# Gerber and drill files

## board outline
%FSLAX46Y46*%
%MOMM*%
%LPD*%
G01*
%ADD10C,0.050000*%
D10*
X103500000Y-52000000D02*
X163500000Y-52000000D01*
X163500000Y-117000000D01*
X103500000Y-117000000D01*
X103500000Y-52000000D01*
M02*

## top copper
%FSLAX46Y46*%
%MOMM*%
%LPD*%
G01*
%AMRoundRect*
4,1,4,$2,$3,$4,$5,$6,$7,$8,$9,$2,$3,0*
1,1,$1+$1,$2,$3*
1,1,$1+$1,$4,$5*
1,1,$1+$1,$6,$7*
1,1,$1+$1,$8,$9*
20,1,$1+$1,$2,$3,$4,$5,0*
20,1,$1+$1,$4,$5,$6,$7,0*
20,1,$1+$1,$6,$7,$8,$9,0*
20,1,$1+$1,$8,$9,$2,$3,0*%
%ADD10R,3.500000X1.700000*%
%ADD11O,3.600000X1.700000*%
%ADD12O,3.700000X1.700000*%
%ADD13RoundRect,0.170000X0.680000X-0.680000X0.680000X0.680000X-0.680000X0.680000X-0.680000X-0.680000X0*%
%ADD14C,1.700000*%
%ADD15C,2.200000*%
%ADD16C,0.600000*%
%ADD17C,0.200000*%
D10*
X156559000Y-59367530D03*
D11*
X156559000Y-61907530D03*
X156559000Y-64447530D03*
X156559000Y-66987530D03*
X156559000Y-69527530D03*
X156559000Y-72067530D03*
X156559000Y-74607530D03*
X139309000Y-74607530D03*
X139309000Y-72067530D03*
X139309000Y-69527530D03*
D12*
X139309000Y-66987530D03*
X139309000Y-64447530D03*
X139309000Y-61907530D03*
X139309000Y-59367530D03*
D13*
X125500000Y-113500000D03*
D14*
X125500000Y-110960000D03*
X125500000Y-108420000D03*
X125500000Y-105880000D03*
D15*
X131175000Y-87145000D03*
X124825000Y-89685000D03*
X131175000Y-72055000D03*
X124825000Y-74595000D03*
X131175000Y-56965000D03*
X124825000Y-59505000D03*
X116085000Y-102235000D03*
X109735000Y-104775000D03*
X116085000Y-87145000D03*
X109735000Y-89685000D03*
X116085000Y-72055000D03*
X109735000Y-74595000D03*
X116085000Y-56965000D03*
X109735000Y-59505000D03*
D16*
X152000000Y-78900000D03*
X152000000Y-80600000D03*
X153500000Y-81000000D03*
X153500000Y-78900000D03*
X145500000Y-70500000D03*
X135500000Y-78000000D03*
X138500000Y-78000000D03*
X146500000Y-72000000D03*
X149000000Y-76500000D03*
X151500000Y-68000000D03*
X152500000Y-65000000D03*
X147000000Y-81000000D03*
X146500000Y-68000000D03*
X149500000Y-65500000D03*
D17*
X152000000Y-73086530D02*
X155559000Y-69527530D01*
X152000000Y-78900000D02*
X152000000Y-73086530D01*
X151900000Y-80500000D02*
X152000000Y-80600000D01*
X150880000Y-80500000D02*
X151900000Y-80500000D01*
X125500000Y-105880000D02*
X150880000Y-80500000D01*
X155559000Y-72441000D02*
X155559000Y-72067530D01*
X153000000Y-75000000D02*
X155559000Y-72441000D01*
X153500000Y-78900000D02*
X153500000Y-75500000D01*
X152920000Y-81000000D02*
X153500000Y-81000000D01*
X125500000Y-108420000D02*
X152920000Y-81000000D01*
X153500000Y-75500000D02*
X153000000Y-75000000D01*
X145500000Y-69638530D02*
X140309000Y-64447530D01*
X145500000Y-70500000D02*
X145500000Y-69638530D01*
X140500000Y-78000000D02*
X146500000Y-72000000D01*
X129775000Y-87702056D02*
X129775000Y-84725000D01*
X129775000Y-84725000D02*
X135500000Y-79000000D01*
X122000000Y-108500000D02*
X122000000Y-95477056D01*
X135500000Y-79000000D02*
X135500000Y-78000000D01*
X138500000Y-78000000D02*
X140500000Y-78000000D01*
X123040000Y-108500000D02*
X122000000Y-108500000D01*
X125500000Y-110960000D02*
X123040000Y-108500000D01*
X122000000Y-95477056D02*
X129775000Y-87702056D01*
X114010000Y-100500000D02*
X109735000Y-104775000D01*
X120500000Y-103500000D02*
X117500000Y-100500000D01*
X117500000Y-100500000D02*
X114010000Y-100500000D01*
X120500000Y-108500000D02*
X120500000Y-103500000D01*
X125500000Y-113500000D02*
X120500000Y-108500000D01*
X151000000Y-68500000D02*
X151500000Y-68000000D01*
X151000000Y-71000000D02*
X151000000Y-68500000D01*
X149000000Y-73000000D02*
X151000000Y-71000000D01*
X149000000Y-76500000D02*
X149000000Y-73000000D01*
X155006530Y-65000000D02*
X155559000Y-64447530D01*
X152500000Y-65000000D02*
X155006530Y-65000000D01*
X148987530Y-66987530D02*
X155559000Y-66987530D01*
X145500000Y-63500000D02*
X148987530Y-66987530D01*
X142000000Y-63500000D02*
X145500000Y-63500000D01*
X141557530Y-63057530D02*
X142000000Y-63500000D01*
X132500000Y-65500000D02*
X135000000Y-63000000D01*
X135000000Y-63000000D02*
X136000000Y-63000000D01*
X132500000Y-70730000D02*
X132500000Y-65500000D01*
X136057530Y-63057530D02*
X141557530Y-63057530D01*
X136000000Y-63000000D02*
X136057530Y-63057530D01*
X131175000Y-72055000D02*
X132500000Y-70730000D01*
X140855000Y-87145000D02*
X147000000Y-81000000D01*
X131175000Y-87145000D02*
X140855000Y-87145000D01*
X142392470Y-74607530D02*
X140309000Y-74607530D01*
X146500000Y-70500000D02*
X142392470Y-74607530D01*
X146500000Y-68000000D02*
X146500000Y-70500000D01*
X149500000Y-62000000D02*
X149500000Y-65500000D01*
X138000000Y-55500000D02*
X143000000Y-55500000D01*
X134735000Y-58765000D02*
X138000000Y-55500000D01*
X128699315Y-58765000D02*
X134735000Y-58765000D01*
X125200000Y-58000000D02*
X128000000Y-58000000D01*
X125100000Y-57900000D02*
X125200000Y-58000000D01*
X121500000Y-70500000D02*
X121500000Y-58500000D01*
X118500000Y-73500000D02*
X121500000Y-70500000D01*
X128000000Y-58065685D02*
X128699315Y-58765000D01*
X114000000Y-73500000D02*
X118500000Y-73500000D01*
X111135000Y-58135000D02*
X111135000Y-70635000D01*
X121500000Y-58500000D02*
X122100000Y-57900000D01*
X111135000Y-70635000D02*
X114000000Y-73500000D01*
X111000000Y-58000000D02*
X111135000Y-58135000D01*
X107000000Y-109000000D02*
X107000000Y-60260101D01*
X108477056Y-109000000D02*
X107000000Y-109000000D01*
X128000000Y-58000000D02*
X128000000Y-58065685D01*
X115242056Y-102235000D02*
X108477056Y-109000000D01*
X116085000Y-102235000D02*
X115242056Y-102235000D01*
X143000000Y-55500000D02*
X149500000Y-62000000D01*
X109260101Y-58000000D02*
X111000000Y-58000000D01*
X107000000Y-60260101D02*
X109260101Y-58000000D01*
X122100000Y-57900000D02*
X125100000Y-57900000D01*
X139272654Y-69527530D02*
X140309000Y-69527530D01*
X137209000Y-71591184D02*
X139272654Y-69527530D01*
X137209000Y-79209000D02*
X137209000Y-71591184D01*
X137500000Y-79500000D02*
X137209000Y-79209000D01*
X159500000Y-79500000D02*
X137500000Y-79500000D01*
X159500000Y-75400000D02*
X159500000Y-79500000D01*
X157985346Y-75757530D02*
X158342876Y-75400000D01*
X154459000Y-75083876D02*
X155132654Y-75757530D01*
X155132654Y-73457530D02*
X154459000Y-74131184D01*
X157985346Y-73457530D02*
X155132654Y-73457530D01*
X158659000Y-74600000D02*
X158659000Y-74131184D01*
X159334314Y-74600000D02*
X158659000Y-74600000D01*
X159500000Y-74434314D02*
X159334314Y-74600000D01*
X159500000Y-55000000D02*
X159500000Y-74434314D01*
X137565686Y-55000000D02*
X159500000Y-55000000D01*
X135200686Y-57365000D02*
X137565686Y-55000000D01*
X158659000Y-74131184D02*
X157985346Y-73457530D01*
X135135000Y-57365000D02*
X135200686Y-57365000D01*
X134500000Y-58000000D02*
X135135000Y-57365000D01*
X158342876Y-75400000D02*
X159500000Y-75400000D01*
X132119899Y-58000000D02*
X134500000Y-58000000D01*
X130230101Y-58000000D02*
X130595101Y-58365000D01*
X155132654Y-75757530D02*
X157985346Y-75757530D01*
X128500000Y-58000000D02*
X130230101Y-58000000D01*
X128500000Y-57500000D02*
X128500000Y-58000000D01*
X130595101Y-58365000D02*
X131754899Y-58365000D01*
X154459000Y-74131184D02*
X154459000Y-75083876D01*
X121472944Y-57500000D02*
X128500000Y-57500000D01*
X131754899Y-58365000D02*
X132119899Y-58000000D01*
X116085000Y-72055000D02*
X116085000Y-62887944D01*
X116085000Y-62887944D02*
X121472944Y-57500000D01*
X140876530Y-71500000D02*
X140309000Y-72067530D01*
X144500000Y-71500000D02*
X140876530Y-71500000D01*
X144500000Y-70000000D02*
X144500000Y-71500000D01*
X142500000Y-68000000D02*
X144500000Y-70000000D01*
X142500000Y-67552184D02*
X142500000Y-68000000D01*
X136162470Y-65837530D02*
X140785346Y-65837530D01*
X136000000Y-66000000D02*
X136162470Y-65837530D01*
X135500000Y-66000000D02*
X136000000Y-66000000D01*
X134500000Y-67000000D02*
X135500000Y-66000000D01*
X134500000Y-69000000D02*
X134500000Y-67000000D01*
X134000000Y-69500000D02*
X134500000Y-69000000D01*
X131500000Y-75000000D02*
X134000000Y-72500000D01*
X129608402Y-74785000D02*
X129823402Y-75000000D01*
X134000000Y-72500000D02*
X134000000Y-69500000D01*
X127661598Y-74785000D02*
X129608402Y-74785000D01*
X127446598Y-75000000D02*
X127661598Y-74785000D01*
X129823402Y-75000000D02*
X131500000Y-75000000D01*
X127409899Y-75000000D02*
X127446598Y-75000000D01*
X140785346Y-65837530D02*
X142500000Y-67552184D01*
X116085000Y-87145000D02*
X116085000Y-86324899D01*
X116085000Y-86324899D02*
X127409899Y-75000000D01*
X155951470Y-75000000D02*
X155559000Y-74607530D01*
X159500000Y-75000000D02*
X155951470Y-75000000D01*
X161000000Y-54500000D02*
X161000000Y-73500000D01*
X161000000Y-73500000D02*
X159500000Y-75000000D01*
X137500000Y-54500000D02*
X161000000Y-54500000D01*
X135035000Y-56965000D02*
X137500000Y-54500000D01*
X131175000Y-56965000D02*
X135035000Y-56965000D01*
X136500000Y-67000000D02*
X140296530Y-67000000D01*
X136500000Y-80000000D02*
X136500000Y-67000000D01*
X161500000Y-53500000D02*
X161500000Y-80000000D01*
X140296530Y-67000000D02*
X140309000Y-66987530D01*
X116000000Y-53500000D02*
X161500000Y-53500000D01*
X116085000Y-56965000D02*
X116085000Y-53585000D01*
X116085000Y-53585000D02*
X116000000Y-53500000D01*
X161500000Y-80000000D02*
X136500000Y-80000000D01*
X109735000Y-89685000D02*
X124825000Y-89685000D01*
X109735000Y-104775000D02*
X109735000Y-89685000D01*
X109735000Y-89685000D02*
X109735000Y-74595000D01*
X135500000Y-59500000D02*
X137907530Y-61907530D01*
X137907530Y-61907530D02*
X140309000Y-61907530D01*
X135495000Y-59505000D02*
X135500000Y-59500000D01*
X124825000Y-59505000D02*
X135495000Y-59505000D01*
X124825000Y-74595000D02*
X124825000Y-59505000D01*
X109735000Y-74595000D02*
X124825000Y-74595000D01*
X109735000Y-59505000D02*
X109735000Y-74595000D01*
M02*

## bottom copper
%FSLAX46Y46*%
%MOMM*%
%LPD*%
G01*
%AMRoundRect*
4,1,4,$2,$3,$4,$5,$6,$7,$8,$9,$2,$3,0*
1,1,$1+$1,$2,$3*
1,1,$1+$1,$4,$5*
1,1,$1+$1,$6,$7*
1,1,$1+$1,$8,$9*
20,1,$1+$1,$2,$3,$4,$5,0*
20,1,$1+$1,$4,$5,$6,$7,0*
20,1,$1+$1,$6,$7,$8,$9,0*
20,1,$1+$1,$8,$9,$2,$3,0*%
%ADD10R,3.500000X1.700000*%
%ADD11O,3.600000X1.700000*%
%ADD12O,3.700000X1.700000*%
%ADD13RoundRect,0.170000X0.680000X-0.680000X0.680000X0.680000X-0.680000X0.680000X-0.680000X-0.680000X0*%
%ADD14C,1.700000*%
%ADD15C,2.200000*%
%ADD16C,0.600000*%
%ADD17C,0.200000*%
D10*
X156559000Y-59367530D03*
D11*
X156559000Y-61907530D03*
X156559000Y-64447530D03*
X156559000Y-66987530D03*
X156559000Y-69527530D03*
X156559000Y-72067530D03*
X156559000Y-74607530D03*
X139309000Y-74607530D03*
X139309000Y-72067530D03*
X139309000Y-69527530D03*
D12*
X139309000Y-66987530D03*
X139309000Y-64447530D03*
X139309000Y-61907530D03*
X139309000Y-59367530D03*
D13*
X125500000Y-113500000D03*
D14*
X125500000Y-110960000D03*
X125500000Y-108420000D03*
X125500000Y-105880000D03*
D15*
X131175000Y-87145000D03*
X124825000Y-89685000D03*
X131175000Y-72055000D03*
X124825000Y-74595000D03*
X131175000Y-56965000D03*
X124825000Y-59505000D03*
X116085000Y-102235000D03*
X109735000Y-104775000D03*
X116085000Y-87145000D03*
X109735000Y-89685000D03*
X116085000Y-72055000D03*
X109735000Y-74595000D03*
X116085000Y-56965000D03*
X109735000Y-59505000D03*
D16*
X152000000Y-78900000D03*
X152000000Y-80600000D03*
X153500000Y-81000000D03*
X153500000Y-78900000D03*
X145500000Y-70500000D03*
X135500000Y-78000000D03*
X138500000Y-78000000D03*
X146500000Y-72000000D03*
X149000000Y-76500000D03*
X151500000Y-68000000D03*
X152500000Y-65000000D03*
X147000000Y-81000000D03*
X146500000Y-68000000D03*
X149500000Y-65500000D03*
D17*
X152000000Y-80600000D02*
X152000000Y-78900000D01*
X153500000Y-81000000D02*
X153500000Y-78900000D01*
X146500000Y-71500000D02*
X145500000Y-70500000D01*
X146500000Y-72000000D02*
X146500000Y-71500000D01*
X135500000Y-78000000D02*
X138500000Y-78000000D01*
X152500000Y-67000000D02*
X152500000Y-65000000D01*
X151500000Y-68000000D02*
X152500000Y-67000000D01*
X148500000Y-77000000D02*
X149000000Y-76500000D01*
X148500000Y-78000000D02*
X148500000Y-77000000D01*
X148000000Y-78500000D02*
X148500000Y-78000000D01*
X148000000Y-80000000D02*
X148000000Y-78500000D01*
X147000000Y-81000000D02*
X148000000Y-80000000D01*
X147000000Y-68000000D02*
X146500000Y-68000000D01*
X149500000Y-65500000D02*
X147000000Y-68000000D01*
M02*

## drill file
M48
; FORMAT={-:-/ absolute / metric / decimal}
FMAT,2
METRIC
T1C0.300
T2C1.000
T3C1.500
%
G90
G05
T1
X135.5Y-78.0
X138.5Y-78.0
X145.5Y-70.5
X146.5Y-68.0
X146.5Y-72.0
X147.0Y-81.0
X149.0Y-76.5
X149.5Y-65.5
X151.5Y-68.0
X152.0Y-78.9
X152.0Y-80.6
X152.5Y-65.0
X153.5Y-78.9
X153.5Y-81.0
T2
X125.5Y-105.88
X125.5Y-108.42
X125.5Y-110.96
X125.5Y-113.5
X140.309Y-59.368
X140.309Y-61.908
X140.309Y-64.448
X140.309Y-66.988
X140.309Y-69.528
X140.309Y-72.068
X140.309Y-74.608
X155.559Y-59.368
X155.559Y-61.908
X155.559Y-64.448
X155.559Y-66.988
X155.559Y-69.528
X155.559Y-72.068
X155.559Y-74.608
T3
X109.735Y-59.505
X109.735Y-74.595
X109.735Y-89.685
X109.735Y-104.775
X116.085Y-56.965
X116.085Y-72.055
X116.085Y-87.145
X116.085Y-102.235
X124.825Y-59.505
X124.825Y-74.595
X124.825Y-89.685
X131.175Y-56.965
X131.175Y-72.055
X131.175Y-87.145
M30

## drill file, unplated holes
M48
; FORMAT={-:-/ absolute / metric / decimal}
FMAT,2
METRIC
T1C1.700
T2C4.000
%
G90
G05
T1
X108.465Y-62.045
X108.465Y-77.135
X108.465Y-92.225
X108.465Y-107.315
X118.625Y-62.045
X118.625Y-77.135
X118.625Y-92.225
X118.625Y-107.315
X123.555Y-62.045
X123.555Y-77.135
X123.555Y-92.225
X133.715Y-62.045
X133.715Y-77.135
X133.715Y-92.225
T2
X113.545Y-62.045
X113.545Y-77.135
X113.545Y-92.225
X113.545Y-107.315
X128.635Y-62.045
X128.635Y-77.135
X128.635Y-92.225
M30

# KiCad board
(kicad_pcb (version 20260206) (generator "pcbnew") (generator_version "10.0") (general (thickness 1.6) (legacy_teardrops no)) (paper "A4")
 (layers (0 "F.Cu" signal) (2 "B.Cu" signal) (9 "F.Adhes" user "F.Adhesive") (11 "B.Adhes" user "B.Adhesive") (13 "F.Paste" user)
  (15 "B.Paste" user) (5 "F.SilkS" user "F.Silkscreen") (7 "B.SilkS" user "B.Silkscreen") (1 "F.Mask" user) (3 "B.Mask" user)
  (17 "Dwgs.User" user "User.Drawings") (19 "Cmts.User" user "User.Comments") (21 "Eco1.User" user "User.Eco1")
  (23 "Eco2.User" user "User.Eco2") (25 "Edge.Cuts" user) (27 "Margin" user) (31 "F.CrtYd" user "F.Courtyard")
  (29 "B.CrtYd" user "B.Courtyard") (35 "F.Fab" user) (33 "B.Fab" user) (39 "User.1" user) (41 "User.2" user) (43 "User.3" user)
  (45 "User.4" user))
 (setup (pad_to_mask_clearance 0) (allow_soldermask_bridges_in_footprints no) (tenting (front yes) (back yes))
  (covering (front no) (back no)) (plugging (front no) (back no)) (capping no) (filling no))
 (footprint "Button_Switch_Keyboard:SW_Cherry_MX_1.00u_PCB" (layer "F.Cu") (at 131.175 56.965)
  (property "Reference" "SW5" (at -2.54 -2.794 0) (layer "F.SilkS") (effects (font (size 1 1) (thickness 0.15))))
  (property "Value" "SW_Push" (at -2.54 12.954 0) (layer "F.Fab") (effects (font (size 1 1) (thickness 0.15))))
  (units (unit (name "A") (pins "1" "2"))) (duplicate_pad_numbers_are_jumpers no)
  (pad "" np_thru_hole circle (at -7.62 5.08) (size 1.7 1.7) (drill 1.7) (layers "*.Cu" "*.Mask"))
  (pad "" np_thru_hole circle (at -2.54 5.08) (size 4 4) (drill 4) (layers "*.Cu" "*.Mask"))
  (pad "" np_thru_hole circle (at 2.54 5.08) (size 1.7 1.7) (drill 1.7) (layers "*.Cu" "*.Mask"))
  (pad "1" thru_hole circle (at 0 0) (size 2.2 2.2) (drill 1.5) (layers "*.Cu" "*.Mask") (remove_unused_layers no)
   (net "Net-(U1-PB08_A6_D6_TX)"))
  (pad "2" thru_hole circle (at -6.35 2.54) (size 2.2 2.2) (drill 1.5) (layers "*.Cu" "*.Mask") (remove_unused_layers no) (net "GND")))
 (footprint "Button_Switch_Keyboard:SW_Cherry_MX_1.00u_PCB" (layer "F.Cu") (at 116.085 72.055)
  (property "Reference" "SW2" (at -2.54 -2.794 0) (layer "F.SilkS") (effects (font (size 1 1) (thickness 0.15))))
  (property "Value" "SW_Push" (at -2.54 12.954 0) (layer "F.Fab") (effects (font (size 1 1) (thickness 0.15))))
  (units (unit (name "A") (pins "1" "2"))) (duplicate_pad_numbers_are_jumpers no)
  (pad "" np_thru_hole circle (at -7.62 5.08) (size 1.7 1.7) (drill 1.7) (layers "*.Cu" "*.Mask"))
  (pad "" np_thru_hole circle (at -2.54 5.08) (size 4 4) (drill 4) (layers "*.Cu" "*.Mask"))
  (pad "" np_thru_hole circle (at 2.54 5.08) (size 1.7 1.7) (drill 1.7) (layers "*.Cu" "*.Mask"))
  (pad "1" thru_hole circle (at 0 0) (size 2.2 2.2) (drill 1.5) (layers "*.Cu" "*.Mask") (remove_unused_layers no)
   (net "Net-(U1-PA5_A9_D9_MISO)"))
  (pad "2" thru_hole circle (at -6.35 2.54) (size 2.2 2.2) (drill 1.5) (layers "*.Cu" "*.Mask") (remove_unused_layers no) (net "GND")))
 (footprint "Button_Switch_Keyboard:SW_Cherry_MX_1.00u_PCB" (layer "F.Cu") (at 116.085 56.965)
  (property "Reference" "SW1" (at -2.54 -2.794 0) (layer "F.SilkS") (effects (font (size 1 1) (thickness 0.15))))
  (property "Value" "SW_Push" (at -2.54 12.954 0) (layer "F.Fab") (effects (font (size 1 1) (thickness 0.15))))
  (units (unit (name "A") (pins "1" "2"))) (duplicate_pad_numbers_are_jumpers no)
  (pad "" np_thru_hole circle (at -7.62 5.08) (size 1.7 1.7) (drill 1.7) (layers "*.Cu" "*.Mask"))
  (pad "" np_thru_hole circle (at -2.54 5.08) (size 4 4) (drill 4) (layers "*.Cu" "*.Mask"))
  (pad "" np_thru_hole circle (at 2.54 5.08) (size 1.7 1.7) (drill 1.7) (layers "*.Cu" "*.Mask"))
  (pad "1" thru_hole circle (at 0 0) (size 2.2 2.2) (drill 1.5) (layers "*.Cu" "*.Mask") (remove_unused_layers no)
   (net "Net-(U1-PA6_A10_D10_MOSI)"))
  (pad "2" thru_hole circle (at -6.35 2.54) (size 2.2 2.2) (drill 1.5) (layers "*.Cu" "*.Mask") (remove_unused_layers no) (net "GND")))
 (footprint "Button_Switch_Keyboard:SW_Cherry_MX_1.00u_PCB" (layer "F.Cu") (at 131.175 87.145)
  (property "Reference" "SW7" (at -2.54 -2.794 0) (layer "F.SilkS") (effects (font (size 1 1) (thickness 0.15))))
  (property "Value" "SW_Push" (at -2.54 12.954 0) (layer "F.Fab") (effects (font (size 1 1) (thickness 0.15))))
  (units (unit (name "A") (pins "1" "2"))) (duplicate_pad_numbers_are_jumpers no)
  (pad "" np_thru_hole circle (at -7.62 5.08) (size 1.7 1.7) (drill 1.7) (layers "*.Cu" "*.Mask"))
  (pad "" np_thru_hole circle (at -2.54 5.08) (size 4 4) (drill 4) (layers "*.Cu" "*.Mask"))
  (pad "" np_thru_hole circle (at 2.54 5.08) (size 1.7 1.7) (drill 1.7) (layers "*.Cu" "*.Mask"))
  (pad "1" thru_hole circle (at 0 0) (size 2.2 2.2) (drill 1.5) (layers "*.Cu" "*.Mask") (remove_unused_layers no)
   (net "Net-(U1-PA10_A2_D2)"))
  (pad "2" thru_hole circle (at -6.35 2.54) (size 2.2 2.2) (drill 1.5) (layers "*.Cu" "*.Mask") (remove_unused_layers no) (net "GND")))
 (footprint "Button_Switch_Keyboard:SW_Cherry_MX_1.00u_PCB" (layer "F.Cu") (at 116.085 102.235)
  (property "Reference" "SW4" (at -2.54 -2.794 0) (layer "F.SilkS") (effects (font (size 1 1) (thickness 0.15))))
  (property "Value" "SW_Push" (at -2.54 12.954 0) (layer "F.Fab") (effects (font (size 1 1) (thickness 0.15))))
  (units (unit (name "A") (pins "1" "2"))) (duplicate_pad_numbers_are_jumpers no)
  (pad "" np_thru_hole circle (at -7.62 5.08) (size 1.7 1.7) (drill 1.7) (layers "*.Cu" "*.Mask"))
  (pad "" np_thru_hole circle (at -2.54 5.08) (size 4 4) (drill 4) (layers "*.Cu" "*.Mask"))
  (pad "" np_thru_hole circle (at 2.54 5.08) (size 1.7 1.7) (drill 1.7) (layers "*.Cu" "*.Mask"))
  (pad "1" thru_hole circle (at 0 0) (size 2.2 2.2) (drill 1.5) (layers "*.Cu" "*.Mask") (remove_unused_layers no)
   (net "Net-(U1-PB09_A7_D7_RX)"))
  (pad "2" thru_hole circle (at -6.35 2.54) (size 2.2 2.2) (drill 1.5) (layers "*.Cu" "*.Mask") (remove_unused_layers no) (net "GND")))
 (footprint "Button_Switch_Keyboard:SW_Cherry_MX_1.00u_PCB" (layer "F.Cu") (at 131.175 72.055)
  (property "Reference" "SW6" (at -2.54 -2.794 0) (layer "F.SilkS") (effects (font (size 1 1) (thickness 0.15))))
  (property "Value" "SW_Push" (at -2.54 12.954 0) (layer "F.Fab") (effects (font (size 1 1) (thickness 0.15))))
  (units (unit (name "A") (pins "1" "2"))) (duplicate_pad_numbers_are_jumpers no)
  (pad "" np_thru_hole circle (at -7.62 5.08) (size 1.7 1.7) (drill 1.7) (layers "*.Cu" "*.Mask"))
  (pad "" np_thru_hole circle (at -2.54 5.08) (size 4 4) (drill 4) (layers "*.Cu" "*.Mask"))
  (pad "" np_thru_hole circle (at 2.54 5.08) (size 1.7 1.7) (drill 1.7) (layers "*.Cu" "*.Mask"))
  (pad "1" thru_hole circle (at 0 0) (size 2.2 2.2) (drill 1.5) (layers "*.Cu" "*.Mask") (remove_unused_layers no)
   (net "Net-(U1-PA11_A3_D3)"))
  (pad "2" thru_hole circle (at -6.35 2.54) (size 2.2 2.2) (drill 1.5) (layers "*.Cu" "*.Mask") (remove_unused_layers no) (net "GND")))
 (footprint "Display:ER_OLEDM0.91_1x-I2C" (layer "F.Cu") (at 125.5 113.5 90)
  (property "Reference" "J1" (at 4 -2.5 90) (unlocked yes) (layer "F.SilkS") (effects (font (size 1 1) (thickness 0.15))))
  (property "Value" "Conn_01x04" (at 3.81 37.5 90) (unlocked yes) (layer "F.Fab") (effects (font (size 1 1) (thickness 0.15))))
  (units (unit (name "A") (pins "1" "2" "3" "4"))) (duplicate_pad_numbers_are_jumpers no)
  (pad "1" thru_hole roundrect (at 0 0 90) (size 1.7 1.7) (drill 1) (layers "*.Cu" "*.Mask") (remove_unused_layers no)
   (roundrect_rratio 0.1) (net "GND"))
  (pad "2" thru_hole circle (at 2.54 0 90) (size 1.7 1.7) (drill 1) (layers "*.Cu" "*.Mask") (remove_unused_layers no)
   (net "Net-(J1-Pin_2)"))
  (pad "3" thru_hole circle (at 5.08 0 90) (size 1.7 1.7) (drill 1) (layers "*.Cu" "*.Mask") (remove_unused_layers no)
   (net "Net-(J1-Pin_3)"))
  (pad "4" thru_hole circle (at 7.62 0 90) (size 1.7 1.7) (drill 1) (layers "*.Cu" "*.Mask") (remove_unused_layers no)
   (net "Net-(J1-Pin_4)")))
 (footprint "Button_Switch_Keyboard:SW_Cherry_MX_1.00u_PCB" (layer "F.Cu") (at 116.085 87.145)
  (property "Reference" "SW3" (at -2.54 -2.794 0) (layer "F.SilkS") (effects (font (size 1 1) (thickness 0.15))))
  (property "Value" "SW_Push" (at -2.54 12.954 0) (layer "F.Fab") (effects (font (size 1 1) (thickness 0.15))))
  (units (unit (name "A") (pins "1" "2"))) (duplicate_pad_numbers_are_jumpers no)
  (pad "" np_thru_hole circle (at -7.62 5.08) (size 1.7 1.7) (drill 1.7) (layers "*.Cu" "*.Mask"))
  (pad "" np_thru_hole circle (at -2.54 5.08) (size 4 4) (drill 4) (layers "*.Cu" "*.Mask"))
  (pad "" np_thru_hole circle (at 2.54 5.08) (size 1.7 1.7) (drill 1.7) (layers "*.Cu" "*.Mask"))
  (pad "1" thru_hole circle (at 0 0) (size 2.2 2.2) (drill 1.5) (layers "*.Cu" "*.Mask") (remove_unused_layers no)
   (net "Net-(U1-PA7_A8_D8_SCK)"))
  (pad "2" thru_hole circle (at -6.35 2.54) (size 2.2 2.2) (drill 1.5) (layers "*.Cu" "*.Mask") (remove_unused_layers no) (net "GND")))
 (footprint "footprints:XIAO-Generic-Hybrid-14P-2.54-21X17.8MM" (layer "B.Cu") (at 147.934 66.98753 180)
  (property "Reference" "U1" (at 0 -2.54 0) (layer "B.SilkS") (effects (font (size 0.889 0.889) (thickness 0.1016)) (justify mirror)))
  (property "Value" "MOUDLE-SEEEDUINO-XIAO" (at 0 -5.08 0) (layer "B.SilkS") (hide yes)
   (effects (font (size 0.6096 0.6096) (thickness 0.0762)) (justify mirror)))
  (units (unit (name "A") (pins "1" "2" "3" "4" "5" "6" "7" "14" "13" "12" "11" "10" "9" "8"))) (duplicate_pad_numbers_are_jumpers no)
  (pad "1" thru_hole rect (at -7.625 7.62 180) (size 3.5 1.7) (drill 1 (offset -1 0)) (layers "*.Cu" "*.Mask") (remove_unused_layers no)
   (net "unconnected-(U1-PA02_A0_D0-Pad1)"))
  (pad "2" thru_hole oval (at -7.625 5.08 180) (size 3.6 1.7) (drill 1 (offset -1 0)) (layers "*.Cu" "*.Mask") (remove_unused_layers no)
   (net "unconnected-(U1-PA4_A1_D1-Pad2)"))
  (pad "3" thru_hole oval (at -7.625 2.54 180) (size 3.6 1.7) (drill 1 (offset -1 0)) (layers "*.Cu" "*.Mask") (remove_unused_layers no)
   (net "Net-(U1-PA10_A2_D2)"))
  (pad "4" thru_hole oval (at -7.625 0 180) (size 3.6 1.7) (drill 1 (offset -1 0)) (layers "*.Cu" "*.Mask") (remove_unused_layers no)
   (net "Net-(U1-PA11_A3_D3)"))
  (pad "5" thru_hole oval (at -7.625 -2.54 180) (size 3.6 1.7) (drill 1 (offset -1 0)) (layers "*.Cu" "*.Mask") (remove_unused_layers no)
   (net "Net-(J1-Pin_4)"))
  (pad "6" thru_hole oval (at -7.625 -5.08) (size 3.6 1.7) (drill 1 (offset 1 0)) (layers "*.Cu" "*.Mask") (remove_unused_layers no)
   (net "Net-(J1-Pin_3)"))
  (pad "7" thru_hole oval (at -7.625 -7.62 180) (size 3.6 1.7) (drill 1 (offset -1 0)) (layers "*.Cu" "*.Mask") (remove_unused_layers no)
   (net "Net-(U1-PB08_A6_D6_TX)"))
  (pad "8" thru_hole oval (at 7.625 -7.62 180) (size 3.6 1.7) (drill 1 (offset 1 0)) (layers "*.Cu" "*.Mask") (remove_unused_layers no)
   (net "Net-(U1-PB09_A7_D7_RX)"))
  (pad "9" thru_hole oval (at 7.625 -5.08 180) (size 3.6 1.7) (drill 1 (offset 1 0)) (layers "*.Cu" "*.Mask") (remove_unused_layers no)
   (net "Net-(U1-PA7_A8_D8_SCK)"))
  (pad "10" thru_hole oval (at 7.625 -2.54 180) (size 3.6 1.7) (drill 1 (offset 1 0)) (layers "*.Cu" "*.Mask") (remove_unused_layers no)
   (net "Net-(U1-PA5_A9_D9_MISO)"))
  (pad "11" thru_hole oval (at 7.625 0 180) (size 3.7 1.7) (drill 1 (offset 1 0)) (layers "*.Cu" "*.Mask") (remove_unused_layers no)
   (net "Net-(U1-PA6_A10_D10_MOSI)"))
  (pad "12" thru_hole oval (at 7.625 2.54 180) (size 3.7 1.7) (drill 1 (offset 1 0)) (layers "*.Cu" "*.Mask") (remove_unused_layers no)
   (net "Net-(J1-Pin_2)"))
  (pad "13" thru_hole oval (at 7.625 5.08 180) (size 3.7 1.7) (drill 1 (offset 1 0)) (layers "*.Cu" "*.Mask") (remove_unused_layers no)
   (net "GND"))
  (pad "14" thru_hole oval (at 7.625 7.62 180) (size 3.7 1.7) (drill 1 (offset 1 0)) (layers "*.Cu" "*.Mask") (remove_unused_layers no)
   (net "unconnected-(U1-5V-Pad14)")))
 (gr_rect (start 103.5 52) (end 163.5 117) (stroke (width 0.05) (type default)) (fill no) (layer "Edge.Cuts"))
 (segment (start 114.01 100.5) (end 109.735 104.775) (width 0.2) (layer "F.Cu") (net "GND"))
 (segment (start 109.735 89.685) (end 124.825 89.685) (width 0.2) (layer "F.Cu") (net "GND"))
 (segment (start 135.495 59.505) (end 135.5 59.5) (width 0.2) (layer "F.Cu") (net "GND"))
 (segment (start 125.5 113.5) (end 120.5 108.5) (width 0.2) (layer "F.Cu") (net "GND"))
 (segment (start 124.825 59.505) (end 135.495 59.505) (width 0.2) (layer "F.Cu") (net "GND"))
 (segment (start 117.5 100.5) (end 114.01 100.5) (width 0.2) (layer "F.Cu") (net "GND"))
 (segment (start 120.5 108.5) (end 120.5 103.5) (width 0.2) (layer "F.Cu") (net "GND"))
 (segment (start 109.735 59.505) (end 109.735 74.595) (width 0.2) (layer "F.Cu") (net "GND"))
 (segment (start 135.5 59.5) (end 137.90753 61.90753) (width 0.2) (layer "F.Cu") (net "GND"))
 (segment (start 137.90753 61.90753) (end 140.309 61.90753) (width 0.2) (layer "F.Cu") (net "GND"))
 (segment (start 109.735 74.595) (end 124.825 74.595) (width 0.2) (layer "F.Cu") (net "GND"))
 (segment (start 109.735 104.775) (end 109.735 89.685) (width 0.2) (layer "F.Cu") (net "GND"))
 (segment (start 109.735 89.685) (end 109.735 74.595) (width 0.2) (layer "F.Cu") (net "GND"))
 (segment (start 120.5 103.5) (end 117.5 100.5) (width 0.2) (layer "F.Cu") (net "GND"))
 (segment (start 124.825 74.595) (end 124.825 59.505) (width 0.2) (layer "F.Cu") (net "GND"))
 (segment (start 161.5 53.5) (end 161.5 80) (width 0.2) (layer "F.Cu") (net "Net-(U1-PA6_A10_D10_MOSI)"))
 (segment (start 136.5 80) (end 136.5 67) (width 0.2) (layer "F.Cu") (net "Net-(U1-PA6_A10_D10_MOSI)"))
 (segment (start 140.29653 67) (end 140.309 66.98753) (width 0.2) (layer "F.Cu") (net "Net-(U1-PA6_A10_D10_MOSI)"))
 (segment (start 116.085 53.585) (end 116 53.5) (width 0.2) (layer "F.Cu") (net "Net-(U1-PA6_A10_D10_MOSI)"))
 (segment (start 136.5 67) (end 140.29653 67) (width 0.2) (layer "F.Cu") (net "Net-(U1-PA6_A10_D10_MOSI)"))
 (segment (start 116.085 56.965) (end 116.085 53.585) (width 0.2) (layer "F.Cu") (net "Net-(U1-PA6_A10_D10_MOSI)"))
 (segment (start 161.5 80) (end 136.5 80) (width 0.2) (layer "F.Cu") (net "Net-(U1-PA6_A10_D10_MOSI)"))
 (segment (start 116 53.5) (end 161.5 53.5) (width 0.2) (layer "F.Cu") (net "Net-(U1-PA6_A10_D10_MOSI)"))
 (segment (start 154.459 74.131184) (end 154.459 75.083876) (width 0.2) (layer "F.Cu") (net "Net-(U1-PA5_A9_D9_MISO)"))
 (segment (start 137.209 79.209) (end 137.209 71.591184) (width 0.2) (layer "F.Cu") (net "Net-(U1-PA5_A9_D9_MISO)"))
 (segment (start 131.754899 58.365) (end 132.119899 58) (width 0.2) (layer "F.Cu") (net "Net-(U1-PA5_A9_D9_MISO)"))
 (segment (start 135.135 57.365) (end 135.200686 57.365) (width 0.2) (layer "F.Cu") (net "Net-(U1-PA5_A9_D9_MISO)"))
 (segment (start 116.085 72.055) (end 116.085 62.887944) (width 0.2) (layer "F.Cu") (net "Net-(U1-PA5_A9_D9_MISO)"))
 (segment (start 159.5 55) (end 159.5 74.434314) (width 0.2) (layer "F.Cu") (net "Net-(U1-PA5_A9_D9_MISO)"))
 (segment (start 130.595101 58.365) (end 131.754899 58.365) (width 0.2) (layer "F.Cu") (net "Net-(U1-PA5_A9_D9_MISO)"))
 (segment (start 159.334314 74.6) (end 158.659 74.6) (width 0.2) (layer "F.Cu") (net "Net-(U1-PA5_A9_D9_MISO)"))
 (segment (start 157.985346 75.75753) (end 158.342876 75.4) (width 0.2) (layer "F.Cu") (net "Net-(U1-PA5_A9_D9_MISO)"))
 (segment (start 155.132654 73.45753) (end 154.459 74.131184) (width 0.2) (layer "F.Cu") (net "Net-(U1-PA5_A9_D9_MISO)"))
 (segment (start 159.5 79.5) (end 137.5 79.5) (width 0.2) (layer "F.Cu") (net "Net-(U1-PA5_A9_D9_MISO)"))
 (segment (start 158.659 74.6) (end 158.659 74.131184) (width 0.2) (layer "F.Cu") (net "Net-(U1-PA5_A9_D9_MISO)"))
 (segment (start 154.459 75.083876) (end 155.132654 75.75753) (width 0.2) (layer "F.Cu") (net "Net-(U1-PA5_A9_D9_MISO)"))
 (segment (start 137.209 71.591184) (end 139.272654 69.52753) (width 0.2) (layer "F.Cu") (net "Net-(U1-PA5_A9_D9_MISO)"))
 (segment (start 137.565686 55) (end 159.5 55) (width 0.2) (layer "F.Cu") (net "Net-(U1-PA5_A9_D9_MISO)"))
 (segment (start 130.230101 58) (end 130.595101 58.365) (width 0.2) (layer "F.Cu") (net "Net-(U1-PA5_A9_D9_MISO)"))
 (segment (start 128.5 58) (end 130.230101 58) (width 0.2) (layer "F.Cu") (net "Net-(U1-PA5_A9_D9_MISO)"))
 (segment (start 121.472944 57.5) (end 128.5 57.5) (width 0.2) (layer "F.Cu") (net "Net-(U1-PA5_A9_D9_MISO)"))
 (segment (start 157.985346 73.45753) (end 155.132654 73.45753) (width 0.2) (layer "F.Cu") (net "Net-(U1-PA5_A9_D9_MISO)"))
 (segment (start 159.5 75.4) (end 159.5 79.5) (width 0.2) (layer "F.Cu") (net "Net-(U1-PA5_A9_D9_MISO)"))
 (segment (start 132.119899 58) (end 134.5 58) (width 0.2) (layer "F.Cu") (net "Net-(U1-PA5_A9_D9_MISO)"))
 (segment (start 159.5 74.434314) (end 159.334314 74.6) (width 0.2) (layer "F.Cu") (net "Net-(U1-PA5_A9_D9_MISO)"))
 (segment (start 137.5 79.5) (end 137.209 79.209) (width 0.2) (layer "F.Cu") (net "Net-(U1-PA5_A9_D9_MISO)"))
 (segment (start 139.272654 69.52753) (end 140.309 69.52753) (width 0.2) (layer "F.Cu") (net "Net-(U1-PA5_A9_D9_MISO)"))
 (segment (start 158.659 74.131184) (end 157.985346 73.45753) (width 0.2) (layer "F.Cu") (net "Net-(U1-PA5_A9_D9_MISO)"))
 (segment (start 134.5 58) (end 135.135 57.365) (width 0.2) (layer "F.Cu") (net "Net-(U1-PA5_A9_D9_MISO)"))
 (segment (start 158.342876 75.4) (end 159.5 75.4) (width 0.2) (layer "F.Cu") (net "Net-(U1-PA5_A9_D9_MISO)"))
 (segment (start 135.200686 57.365) (end 137.565686 55) (width 0.2) (layer "F.Cu") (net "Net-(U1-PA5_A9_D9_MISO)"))
 (segment (start 128.5 57.5) (end 128.5 58) (width 0.2) (layer "F.Cu") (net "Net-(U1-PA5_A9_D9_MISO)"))
 (segment (start 155.132654 75.75753) (end 157.985346 75.75753) (width 0.2) (layer "F.Cu") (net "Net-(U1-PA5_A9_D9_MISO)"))
 (segment (start 116.085 62.887944) (end 121.472944 57.5) (width 0.2) (layer "F.Cu") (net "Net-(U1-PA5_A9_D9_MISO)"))
 (segment (start 116.085 86.324899) (end 127.409899 75) (width 0.2) (layer "F.Cu") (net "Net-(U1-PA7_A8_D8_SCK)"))
 (segment (start 134 72.5) (end 134 69.5) (width 0.2) (layer "F.Cu") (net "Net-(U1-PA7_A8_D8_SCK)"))
 (segment (start 142.5 68) (end 144.5 70) (width 0.2) (layer "F.Cu") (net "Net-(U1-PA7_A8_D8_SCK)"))
 (segment (start 129.608402 74.785) (end 129.823402 75) (width 0.2) (layer "F.Cu") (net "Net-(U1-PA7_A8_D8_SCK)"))
 (segment (start 127.661598 74.785) (end 129.608402 74.785) (width 0.2) (layer "F.Cu") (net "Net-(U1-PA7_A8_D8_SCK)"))
 (segment (start 135.5 66) (end 136 66) (width 0.2) (layer "F.Cu") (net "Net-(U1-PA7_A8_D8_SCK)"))
 (segment (start 144.5 71.5) (end 140.87653 71.5) (width 0.2) (layer "F.Cu") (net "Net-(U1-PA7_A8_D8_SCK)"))
 (segment (start 144.5 70) (end 144.5 71.5) (width 0.2) (layer "F.Cu") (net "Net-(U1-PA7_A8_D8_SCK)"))
 (segment (start 131.5 75) (end 134 72.5) (width 0.2) (layer "F.Cu") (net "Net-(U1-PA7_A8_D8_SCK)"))
 (segment (start 142.5 67.552184) (end 142.5 68) (width 0.2) (layer "F.Cu") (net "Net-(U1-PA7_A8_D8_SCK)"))
 (segment (start 129.823402 75) (end 131.5 75) (width 0.2) (layer "F.Cu") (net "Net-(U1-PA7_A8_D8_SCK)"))
 (segment (start 134.5 69) (end 134.5 67) (width 0.2) (layer "F.Cu") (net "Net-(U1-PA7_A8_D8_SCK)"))
 (segment (start 136 66) (end 136.16247 65.83753) (width 0.2) (layer "F.Cu") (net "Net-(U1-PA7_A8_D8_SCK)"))
 (segment (start 140.87653 71.5) (end 140.309 72.06753) (width 0.2) (layer "F.Cu") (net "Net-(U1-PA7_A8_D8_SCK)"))
 (segment (start 116.085 87.145) (end 116.085 86.324899) (width 0.2) (layer "F.Cu") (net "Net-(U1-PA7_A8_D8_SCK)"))
 (segment (start 134.5 67) (end 135.5 66) (width 0.2) (layer "F.Cu") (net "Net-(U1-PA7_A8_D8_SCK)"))
 (segment (start 134 69.5) (end 134.5 69) (width 0.2) (layer "F.Cu") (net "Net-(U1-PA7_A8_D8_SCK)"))
 (segment (start 127.409899 75) (end 127.446598 75) (width 0.2) (layer "F.Cu") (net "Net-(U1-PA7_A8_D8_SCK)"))
 (segment (start 136.16247 65.83753) (end 140.785346 65.83753) (width 0.2) (layer "F.Cu") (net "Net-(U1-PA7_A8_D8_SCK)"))
 (segment (start 140.785346 65.83753) (end 142.5 67.552184) (width 0.2) (layer "F.Cu") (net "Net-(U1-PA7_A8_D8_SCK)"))
 (segment (start 127.446598 75) (end 127.661598 74.785) (width 0.2) (layer "F.Cu") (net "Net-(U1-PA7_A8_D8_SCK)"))
 (segment (start 128.699315 58.765) (end 134.735 58.765) (width 0.2) (layer "F.Cu") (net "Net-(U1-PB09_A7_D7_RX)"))
 (segment (start 111.135 70.635) (end 114 73.5) (width 0.2) (layer "F.Cu") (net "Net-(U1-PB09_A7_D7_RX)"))
 (segment (start 115.242056 102.235) (end 108.477056 109) (width 0.2) (layer "F.Cu") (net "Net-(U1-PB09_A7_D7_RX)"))
 (segment (start 128 58) (end 128 58.065685) (width 0.2) (layer "F.Cu") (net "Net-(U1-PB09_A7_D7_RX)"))
 (segment (start 125.1 57.9) (end 125.2 58) (width 0.2) (layer "F.Cu") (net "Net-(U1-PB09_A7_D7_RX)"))
 (segment (start 149.5 62) (end 149.5 65.5) (width 0.2) (layer "F.Cu") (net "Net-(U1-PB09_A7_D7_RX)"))
 (segment (start 107 60.260101) (end 109.260101 58) (width 0.2) (layer "F.Cu") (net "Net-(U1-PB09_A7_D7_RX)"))
 (segment (start 125.2 58) (end 128 58) (width 0.2) (layer "F.Cu") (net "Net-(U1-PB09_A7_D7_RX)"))
 (segment (start 121.5 58.5) (end 122.1 57.9) (width 0.2) (layer "F.Cu") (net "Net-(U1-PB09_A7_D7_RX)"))
 (segment (start 107 109) (end 107 60.260101) (width 0.2) (layer "F.Cu") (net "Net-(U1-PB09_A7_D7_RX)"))
 (segment (start 109.260101 58) (end 111 58) (width 0.2) (layer "F.Cu") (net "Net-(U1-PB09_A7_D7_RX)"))
 (segment (start 116.085 102.235) (end 115.242056 102.235) (width 0.2) (layer "F.Cu") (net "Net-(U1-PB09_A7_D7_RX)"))
 (segment (start 111 58) (end 111.135 58.135) (width 0.2) (layer "F.Cu") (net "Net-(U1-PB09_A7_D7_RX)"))
 (segment (start 134.735 58.765) (end 138 55.5) (width 0.2) (layer "F.Cu") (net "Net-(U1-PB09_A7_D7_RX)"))
 (segment (start 122.1 57.9) (end 125.1 57.9) (width 0.2) (layer "F.Cu") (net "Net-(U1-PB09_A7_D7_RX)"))
 (segment (start 146.5 70.5) (end 142.39247 74.60753) (width 0.2) (layer "F.Cu") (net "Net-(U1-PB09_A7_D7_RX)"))
 (segment (start 128 58.065685) (end 128.699315 58.765) (width 0.2) (layer "F.Cu") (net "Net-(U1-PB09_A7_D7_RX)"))
 (segment (start 142.39247 74.60753) (end 140.309 74.60753) (width 0.2) (layer "F.Cu") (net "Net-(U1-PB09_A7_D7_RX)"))
 (segment (start 111.135 58.135) (end 111.135 70.635) (width 0.2) (layer "F.Cu") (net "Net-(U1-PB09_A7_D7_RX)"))
 (segment (start 143 55.5) (end 149.5 62) (width 0.2) (layer "F.Cu") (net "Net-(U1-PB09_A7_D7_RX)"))
 (segment (start 114 73.5) (end 118.5 73.5) (width 0.2) (layer "F.Cu") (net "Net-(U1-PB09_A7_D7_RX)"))
 (segment (start 121.5 70.5) (end 121.5 58.5) (width 0.2) (layer "F.Cu") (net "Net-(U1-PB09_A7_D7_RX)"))
 (segment (start 118.5 73.5) (end 121.5 70.5) (width 0.2) (layer "F.Cu") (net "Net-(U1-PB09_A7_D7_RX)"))
 (segment (start 146.5 68) (end 146.5 70.5) (width 0.2) (layer "F.Cu") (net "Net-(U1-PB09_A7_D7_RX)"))
 (segment (start 138 55.5) (end 143 55.5) (width 0.2) (layer "F.Cu") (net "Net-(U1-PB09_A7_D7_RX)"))
 (segment (start 108.477056 109) (end 107 109) (width 0.2) (layer "F.Cu") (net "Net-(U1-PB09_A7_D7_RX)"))
 (via (at 149.5 65.5) (size 0.6) (drill 0.3) (layers "F.Cu" "B.Cu") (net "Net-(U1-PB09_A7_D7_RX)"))
 (via (at 146.5 68) (size 0.6) (drill 0.3) (layers "F.Cu" "B.Cu") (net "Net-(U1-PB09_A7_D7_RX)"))
 (segment (start 149.5 65.5) (end 147 68) (width 0.2) (layer "B.Cu") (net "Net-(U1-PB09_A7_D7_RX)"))
 (segment (start 147 68) (end 146.5 68) (width 0.2) (layer "B.Cu") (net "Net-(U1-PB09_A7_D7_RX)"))
 (segment (start 131.175 56.965) (end 135.035 56.965) (width 0.2) (layer "F.Cu") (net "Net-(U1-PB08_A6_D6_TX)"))
 (segment (start 159.5 75) (end 155.95147 75) (width 0.2) (layer "F.Cu") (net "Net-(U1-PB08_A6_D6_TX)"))
 (segment (start 161 54.5) (end 161 73.5) (width 0.2) (layer "F.Cu") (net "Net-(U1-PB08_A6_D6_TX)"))
 (segment (start 161 73.5) (end 159.5 75) (width 0.2) (layer "F.Cu") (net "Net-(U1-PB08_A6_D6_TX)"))
 (segment (start 137.5 54.5) (end 161 54.5) (width 0.2) (layer "F.Cu") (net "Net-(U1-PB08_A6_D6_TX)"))
 (segment (start 135.035 56.965) (end 137.5 54.5) (width 0.2) (layer "F.Cu") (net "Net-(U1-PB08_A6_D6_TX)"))
 (segment (start 155.95147 75) (end 155.559 74.60753) (width 0.2) (layer "F.Cu") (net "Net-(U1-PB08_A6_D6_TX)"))
 (segment (start 132.5 70.73) (end 132.5 65.5) (width 0.2) (layer "F.Cu") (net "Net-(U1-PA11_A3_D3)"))
 (segment (start 135 63) (end 136 63) (width 0.2) (layer "F.Cu") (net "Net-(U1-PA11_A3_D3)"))
 (segment (start 131.175 72.055) (end 132.5 70.73) (width 0.2) (layer "F.Cu") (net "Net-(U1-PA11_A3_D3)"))
 (segment (start 132.5 65.5) (end 135 63) (width 0.2) (layer "F.Cu") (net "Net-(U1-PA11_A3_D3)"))
 (segment (start 136 63) (end 136.05753 63.05753) (width 0.2) (layer "F.Cu") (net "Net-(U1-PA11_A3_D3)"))
 (segment (start 141.55753 63.05753) (end 142 63.5) (width 0.2) (layer "F.Cu") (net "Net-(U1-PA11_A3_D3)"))
 (segment (start 136.05753 63.05753) (end 141.55753 63.05753) (width 0.2) (layer "F.Cu") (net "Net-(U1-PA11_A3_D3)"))
 (segment (start 145.5 63.5) (end 148.98753 66.98753) (width 0.2) (layer "F.Cu") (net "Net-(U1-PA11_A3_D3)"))
 (segment (start 142 63.5) (end 145.5 63.5) (width 0.2) (layer "F.Cu") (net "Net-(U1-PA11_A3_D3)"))
 (segment (start 148.98753 66.98753) (end 155.559 66.98753) (width 0.2) (layer "F.Cu") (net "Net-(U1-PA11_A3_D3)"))
 (segment (start 151 68.5) (end 151.5 68) (width 0.2) (layer "F.Cu") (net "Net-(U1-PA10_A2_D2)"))
 (segment (start 131.175 87.145) (end 140.855 87.145) (width 0.2) (layer "F.Cu") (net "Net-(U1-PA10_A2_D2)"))
 (segment (start 155.00653 65) (end 155.559 64.44753) (width 0.2) (layer "F.Cu") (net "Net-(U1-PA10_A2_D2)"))
 (segment (start 152.5 65) (end 155.00653 65) (width 0.2) (layer "F.Cu") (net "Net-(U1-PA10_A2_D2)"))
 (segment (start 151 71) (end 151 68.5) (width 0.2) (layer "F.Cu") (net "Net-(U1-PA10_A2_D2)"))
 (segment (start 149 73) (end 151 71) (width 0.2) (layer "F.Cu") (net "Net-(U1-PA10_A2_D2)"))
 (segment (start 140.855 87.145) (end 147 81) (width 0.2) (layer "F.Cu") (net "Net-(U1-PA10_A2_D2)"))
 (segment (start 149 76.5) (end 149 73) (width 0.2) (layer "F.Cu") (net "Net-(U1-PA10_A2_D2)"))
 (via (at 147 81) (size 0.6) (drill 0.3) (layers "F.Cu" "B.Cu") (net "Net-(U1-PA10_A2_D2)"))
 (via (at 151.5 68) (size 0.6) (drill 0.3) (layers "F.Cu" "B.Cu") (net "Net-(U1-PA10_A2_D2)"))
 (via (at 152.5 65) (size 0.6) (drill 0.3) (layers "F.Cu" "B.Cu") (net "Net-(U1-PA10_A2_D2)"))
 (via (at 149 76.5) (size 0.6) (drill 0.3) (layers "F.Cu" "B.Cu") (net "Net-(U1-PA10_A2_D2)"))
 (segment (start 151.5 68) (end 152.5 67) (width 0.2) (layer "B.Cu") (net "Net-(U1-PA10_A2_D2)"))
 (segment (start 152.5 67) (end 152.5 65) (width 0.2) (layer "B.Cu") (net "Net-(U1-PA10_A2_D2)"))
 (segment (start 147 81) (end 148 80) (width 0.2) (layer "B.Cu") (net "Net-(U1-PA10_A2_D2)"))
 (segment (start 148.5 78) (end 148.5 77) (width 0.2) (layer "B.Cu") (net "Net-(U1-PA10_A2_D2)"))
 (segment (start 148 80) (end 148 78.5) (width 0.2) (layer "B.Cu") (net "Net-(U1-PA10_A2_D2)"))
 (segment (start 148.5 77) (end 149 76.5) (width 0.2) (layer "B.Cu") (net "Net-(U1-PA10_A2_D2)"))
 (segment (start 148 78.5) (end 148.5 78) (width 0.2) (layer "B.Cu") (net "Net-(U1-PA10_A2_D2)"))
 (segment (start 145.5 70.5) (end 145.5 69.63853) (width 0.2) (layer "F.Cu") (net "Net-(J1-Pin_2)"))
 (segment (start 138.5 78) (end 140.5 78) (width 0.2) (layer "F.Cu") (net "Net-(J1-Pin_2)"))
 (segment (start 129.775 87.702056) (end 129.775 84.725) (width 0.2) (layer "F.Cu") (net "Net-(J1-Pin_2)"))
 (segment (start 125.5 110.96) (end 123.04 108.5) (width 0.2) (layer "F.Cu") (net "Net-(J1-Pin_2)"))
 (segment (start 122 95.477056) (end 129.775 87.702056) (width 0.2) (layer "F.Cu") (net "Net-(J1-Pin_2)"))
 (segment (start 135.5 79) (end 135.5 78) (width 0.2) (layer "F.Cu") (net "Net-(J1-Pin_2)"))
 (segment (start 129.775 84.725) (end 135.5 79) (width 0.2) (layer "F.Cu") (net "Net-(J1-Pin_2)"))
 (segment (start 140.5 78) (end 146.5 72) (width 0.2) (layer "F.Cu") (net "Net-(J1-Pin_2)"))
 (segment (start 122 108.5) (end 122 95.477056) (width 0.2) (layer "F.Cu") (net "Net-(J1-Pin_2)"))
 (segment (start 145.5 69.63853) (end 140.309 64.44753) (width 0.2) (layer "F.Cu") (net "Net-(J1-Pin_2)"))
 (segment (start 123.04 108.5) (end 122 108.5) (width 0.2) (layer "F.Cu") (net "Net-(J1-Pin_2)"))
 (via (at 145.5 70.5) (size 0.6) (drill 0.3) (layers "F.Cu" "B.Cu") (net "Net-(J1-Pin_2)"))
 (via (at 146.5 72) (size 0.6) (drill 0.3) (layers "F.Cu" "B.Cu") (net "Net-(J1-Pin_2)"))
 (via (at 138.5 78) (size 0.6) (drill 0.3) (layers "F.Cu" "B.Cu") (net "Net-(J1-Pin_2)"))
 (via (at 135.5 78) (size 0.6) (drill 0.3) (layers "F.Cu" "B.Cu") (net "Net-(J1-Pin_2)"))
 (segment (start 135.5 78) (end 138.5 78) (width 0.2) (layer "B.Cu") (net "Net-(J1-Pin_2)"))
 (segment (start 146.5 72) (end 146.5 71.5) (width 0.2) (layer "B.Cu") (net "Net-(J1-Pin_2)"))
 (segment (start 146.5 71.5) (end 145.5 70.5) (width 0.2) (layer "B.Cu") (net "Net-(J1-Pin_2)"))
 (segment (start 153 75) (end 155.559 72.441) (width 0.2) (layer "F.Cu") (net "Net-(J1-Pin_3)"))
 (segment (start 155.559 72.441) (end 155.559 72.06753) (width 0.2) (layer "F.Cu") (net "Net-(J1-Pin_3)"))
 (segment (start 152.92 81) (end 153.5 81) (width 0.2) (layer "F.Cu") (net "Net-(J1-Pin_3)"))
 (segment (start 153.5 78.9) (end 153.5 75.5) (width 0.2) (layer "F.Cu") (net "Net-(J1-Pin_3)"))
 (segment (start 125.5 108.42) (end 152.92 81) (width 0.2) (layer "F.Cu") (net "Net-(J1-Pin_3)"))
 (segment (start 153.5 75.5) (end 153 75) (width 0.2) (layer "F.Cu") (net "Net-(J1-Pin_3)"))
 (via (at 153.5 81) (size 0.6) (drill 0.3) (layers "F.Cu" "B.Cu") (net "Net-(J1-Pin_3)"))
 (via (at 153.5 78.9) (size 0.6) (drill 0.3) (layers "F.Cu" "B.Cu") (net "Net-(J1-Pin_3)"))
 (segment (start 153.5 81) (end 153.5 78.9) (width 0.2) (layer "B.Cu") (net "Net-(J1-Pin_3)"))
 (segment (start 150.88 80.5) (end 151.9 80.5) (width 0.2) (layer "F.Cu") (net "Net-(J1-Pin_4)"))
 (segment (start 152 78.9) (end 152 73.08653) (width 0.2) (layer "F.Cu") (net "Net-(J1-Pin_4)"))
 (segment (start 125.5 105.88) (end 150.88 80.5) (width 0.2) (layer "F.Cu") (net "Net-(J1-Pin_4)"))
 (segment (start 151.9 80.5) (end 152 80.6) (width 0.2) (layer "F.Cu") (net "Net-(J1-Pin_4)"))
 (segment (start 152 73.08653) (end 155.559 69.52753) (width 0.2) (layer "F.Cu") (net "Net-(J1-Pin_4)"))
 (via (at 152 80.6) (size 0.6) (drill 0.3) (layers "F.Cu" "B.Cu") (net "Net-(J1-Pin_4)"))
 (via (at 152 78.9) (size 0.6) (drill 0.3) (layers "F.Cu" "B.Cu") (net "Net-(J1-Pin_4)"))
 (segment (start 152 80.6) (end 152 78.9) (width 0.2) (layer "B.Cu") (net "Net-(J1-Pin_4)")))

